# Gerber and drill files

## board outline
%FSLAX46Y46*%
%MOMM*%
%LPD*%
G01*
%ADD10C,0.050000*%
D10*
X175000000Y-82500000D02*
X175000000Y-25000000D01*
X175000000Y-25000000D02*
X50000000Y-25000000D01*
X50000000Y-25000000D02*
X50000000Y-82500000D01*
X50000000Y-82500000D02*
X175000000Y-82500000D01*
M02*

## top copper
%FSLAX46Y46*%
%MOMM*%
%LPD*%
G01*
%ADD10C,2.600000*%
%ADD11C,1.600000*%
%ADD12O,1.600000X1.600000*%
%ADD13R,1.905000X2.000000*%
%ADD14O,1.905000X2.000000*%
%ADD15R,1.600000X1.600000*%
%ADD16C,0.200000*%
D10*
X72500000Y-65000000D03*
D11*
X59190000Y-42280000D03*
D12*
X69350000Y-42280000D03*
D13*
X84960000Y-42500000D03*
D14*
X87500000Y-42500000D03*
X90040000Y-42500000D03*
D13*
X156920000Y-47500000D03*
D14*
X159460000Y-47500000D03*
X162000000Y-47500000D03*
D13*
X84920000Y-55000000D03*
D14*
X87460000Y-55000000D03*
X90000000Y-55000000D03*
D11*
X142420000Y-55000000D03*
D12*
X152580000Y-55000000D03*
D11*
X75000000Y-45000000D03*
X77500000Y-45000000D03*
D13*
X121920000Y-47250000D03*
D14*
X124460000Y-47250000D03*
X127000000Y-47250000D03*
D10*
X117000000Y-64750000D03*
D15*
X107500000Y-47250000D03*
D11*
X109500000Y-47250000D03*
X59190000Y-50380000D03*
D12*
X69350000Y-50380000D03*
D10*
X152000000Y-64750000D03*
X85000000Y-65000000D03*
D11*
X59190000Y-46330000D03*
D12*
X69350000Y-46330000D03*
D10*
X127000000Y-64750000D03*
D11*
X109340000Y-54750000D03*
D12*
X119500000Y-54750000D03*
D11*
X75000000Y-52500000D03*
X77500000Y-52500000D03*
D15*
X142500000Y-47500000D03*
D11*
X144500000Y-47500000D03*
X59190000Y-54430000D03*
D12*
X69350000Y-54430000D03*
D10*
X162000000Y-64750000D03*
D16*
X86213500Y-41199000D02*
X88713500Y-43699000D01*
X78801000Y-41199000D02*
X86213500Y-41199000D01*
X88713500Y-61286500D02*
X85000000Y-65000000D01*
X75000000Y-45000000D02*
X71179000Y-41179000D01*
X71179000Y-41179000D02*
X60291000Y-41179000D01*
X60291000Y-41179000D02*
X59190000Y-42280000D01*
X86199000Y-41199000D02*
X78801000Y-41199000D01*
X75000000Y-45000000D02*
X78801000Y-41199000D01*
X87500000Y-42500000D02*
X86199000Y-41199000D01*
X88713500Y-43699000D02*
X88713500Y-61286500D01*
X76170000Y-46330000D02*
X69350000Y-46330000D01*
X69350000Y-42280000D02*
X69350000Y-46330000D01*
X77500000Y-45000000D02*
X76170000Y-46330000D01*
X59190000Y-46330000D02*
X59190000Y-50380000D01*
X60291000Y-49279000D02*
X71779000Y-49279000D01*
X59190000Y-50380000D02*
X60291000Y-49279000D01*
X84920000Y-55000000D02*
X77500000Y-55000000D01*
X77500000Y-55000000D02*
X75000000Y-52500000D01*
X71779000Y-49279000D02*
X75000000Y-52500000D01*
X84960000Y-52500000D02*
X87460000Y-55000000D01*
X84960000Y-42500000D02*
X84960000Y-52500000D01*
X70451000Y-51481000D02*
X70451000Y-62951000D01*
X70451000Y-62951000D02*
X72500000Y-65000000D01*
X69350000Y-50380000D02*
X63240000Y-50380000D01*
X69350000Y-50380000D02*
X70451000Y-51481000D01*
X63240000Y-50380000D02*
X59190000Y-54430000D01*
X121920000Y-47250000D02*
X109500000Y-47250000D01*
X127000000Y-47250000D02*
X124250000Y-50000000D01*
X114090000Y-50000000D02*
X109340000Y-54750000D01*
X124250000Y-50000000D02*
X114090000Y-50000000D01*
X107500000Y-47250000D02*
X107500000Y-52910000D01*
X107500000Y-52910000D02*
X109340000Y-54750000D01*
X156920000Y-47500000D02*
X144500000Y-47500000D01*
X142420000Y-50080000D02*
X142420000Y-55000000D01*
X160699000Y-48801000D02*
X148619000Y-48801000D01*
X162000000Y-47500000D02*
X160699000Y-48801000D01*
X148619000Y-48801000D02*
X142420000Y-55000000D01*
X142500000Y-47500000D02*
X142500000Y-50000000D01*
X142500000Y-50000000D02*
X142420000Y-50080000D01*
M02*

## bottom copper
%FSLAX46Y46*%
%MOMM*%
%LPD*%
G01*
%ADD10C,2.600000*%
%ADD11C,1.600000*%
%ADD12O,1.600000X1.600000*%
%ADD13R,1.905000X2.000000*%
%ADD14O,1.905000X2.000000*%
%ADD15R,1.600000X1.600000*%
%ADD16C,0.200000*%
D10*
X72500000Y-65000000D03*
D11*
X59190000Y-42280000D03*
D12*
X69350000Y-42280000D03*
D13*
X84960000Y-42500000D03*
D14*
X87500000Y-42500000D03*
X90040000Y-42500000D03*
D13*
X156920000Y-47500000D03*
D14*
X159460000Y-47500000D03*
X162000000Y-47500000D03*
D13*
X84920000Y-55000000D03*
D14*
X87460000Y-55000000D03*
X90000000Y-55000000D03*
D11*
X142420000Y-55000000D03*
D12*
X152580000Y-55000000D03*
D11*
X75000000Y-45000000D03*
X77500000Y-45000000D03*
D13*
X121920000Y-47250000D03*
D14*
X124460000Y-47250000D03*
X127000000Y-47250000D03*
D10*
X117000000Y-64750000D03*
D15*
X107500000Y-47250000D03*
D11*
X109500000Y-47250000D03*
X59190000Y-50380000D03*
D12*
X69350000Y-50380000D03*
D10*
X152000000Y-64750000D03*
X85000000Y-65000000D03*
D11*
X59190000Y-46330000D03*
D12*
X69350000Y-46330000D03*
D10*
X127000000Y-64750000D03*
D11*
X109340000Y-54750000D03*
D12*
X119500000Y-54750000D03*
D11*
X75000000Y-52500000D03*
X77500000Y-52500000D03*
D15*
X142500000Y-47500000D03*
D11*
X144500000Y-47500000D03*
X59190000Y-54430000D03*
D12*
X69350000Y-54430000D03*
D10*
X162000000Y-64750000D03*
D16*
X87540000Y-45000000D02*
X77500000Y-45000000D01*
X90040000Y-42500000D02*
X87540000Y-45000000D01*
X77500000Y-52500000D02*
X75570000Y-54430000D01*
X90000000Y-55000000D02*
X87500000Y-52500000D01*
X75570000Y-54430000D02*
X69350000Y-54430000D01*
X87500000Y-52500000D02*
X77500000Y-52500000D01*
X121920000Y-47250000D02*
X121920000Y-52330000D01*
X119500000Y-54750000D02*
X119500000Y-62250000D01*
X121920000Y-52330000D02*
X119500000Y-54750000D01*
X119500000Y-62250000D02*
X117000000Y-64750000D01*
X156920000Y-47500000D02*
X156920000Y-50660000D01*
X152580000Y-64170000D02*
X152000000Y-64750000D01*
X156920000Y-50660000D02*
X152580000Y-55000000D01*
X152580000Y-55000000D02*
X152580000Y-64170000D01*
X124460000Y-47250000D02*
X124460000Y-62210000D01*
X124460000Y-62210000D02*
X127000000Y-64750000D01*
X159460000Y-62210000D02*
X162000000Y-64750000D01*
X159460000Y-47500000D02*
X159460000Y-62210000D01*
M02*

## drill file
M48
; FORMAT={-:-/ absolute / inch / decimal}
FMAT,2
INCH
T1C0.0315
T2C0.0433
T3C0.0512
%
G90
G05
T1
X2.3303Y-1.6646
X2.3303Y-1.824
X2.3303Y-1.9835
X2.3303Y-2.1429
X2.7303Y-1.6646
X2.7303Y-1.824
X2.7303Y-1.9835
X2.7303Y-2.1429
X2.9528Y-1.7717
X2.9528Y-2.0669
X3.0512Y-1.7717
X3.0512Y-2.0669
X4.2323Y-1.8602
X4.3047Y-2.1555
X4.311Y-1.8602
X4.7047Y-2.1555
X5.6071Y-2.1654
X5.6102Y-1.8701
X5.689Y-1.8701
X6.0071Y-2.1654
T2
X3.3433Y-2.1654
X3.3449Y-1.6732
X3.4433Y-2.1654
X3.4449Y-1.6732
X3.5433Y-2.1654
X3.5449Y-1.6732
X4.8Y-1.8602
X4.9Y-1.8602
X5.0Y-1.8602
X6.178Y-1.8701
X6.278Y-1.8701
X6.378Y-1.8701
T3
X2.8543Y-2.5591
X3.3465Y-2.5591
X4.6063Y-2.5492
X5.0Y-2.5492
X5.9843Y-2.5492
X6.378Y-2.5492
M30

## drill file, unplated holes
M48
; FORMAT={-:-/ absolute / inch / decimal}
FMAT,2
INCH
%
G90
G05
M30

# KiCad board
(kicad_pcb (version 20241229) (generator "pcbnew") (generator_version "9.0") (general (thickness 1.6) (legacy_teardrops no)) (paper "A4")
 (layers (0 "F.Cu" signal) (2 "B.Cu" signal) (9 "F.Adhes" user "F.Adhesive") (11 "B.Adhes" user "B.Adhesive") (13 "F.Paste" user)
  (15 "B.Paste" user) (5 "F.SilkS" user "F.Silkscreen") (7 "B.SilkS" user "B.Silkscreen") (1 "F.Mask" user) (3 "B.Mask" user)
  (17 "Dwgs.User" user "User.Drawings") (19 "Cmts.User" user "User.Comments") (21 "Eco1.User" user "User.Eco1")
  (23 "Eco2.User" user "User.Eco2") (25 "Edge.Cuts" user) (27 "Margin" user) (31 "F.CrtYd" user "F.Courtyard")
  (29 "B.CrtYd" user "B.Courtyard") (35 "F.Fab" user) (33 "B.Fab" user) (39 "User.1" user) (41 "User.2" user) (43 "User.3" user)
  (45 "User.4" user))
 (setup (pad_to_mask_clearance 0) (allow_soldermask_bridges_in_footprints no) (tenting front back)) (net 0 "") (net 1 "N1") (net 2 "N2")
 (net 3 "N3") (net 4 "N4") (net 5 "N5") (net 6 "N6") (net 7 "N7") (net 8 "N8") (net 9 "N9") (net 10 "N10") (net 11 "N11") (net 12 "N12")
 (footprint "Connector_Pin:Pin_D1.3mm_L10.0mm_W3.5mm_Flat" (layer "F.Cu") (at 72.5 65)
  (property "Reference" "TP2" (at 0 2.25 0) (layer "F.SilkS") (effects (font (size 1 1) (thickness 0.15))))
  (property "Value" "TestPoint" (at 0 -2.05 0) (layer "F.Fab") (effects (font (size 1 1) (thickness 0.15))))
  (pad "1" thru_hole circle (at 0 0) (size 2.6 2.6) (drill 1.3) (layers "*.Cu" "*.Mask") (remove_unused_layers no) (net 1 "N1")))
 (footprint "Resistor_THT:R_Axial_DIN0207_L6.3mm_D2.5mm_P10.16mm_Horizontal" (layer "F.Cu") (at 59.19 42.28)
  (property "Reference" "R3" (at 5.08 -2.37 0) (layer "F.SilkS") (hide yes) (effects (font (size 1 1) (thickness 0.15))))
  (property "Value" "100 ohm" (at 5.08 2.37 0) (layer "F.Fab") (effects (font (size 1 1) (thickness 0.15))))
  (pad "1" thru_hole circle (at 0 0) (size 1.6 1.6) (drill 0.8) (layers "*.Cu" "*.Mask") (remove_unused_layers no) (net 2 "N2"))
  (pad "2" thru_hole oval (at 10.16 0) (size 1.6 1.6) (drill 0.8) (layers "*.Cu" "*.Mask") (remove_unused_layers no) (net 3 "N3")))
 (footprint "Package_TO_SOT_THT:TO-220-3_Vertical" (layer "F.Cu") (at 84.96 42.5)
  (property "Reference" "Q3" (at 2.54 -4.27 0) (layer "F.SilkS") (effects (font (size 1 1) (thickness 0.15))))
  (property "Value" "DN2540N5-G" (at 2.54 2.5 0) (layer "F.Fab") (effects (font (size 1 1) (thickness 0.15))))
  (pad "1" thru_hole rect (at 0 0) (size 1.905 2) (drill 1.1) (layers "*.Cu" "*.Mask") (remove_unused_layers no) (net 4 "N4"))
  (pad "2" thru_hole oval (at 2.54 0) (size 1.905 2) (drill 1.1) (layers "*.Cu" "*.Mask") (remove_unused_layers no) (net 2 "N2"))
  (pad "3" thru_hole oval (at 5.08 0) (size 1.905 2) (drill 1.1) (layers "*.Cu" "*.Mask") (remove_unused_layers no) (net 3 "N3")))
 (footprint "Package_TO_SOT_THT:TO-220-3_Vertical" (layer "F.Cu") (at 156.92 47.5)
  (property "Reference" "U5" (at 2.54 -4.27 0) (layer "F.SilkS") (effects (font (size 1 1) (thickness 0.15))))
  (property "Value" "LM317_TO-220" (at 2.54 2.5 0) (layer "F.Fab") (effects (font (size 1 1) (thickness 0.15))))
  (pad "1" thru_hole rect (at 0 0) (size 1.905 2) (drill 1.1) (layers "*.Cu" "*.Mask") (remove_unused_layers no) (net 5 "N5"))
  (pad "2" thru_hole oval (at 2.54 0) (size 1.905 2) (drill 1.1) (layers "*.Cu" "*.Mask") (remove_unused_layers no) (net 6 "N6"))
  (pad "3" thru_hole oval (at 5.08 0) (size 1.905 2) (drill 1.1) (layers "*.Cu" "*.Mask") (remove_unused_layers no) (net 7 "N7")))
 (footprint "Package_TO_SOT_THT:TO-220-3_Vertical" (layer "F.Cu") (at 84.92 55)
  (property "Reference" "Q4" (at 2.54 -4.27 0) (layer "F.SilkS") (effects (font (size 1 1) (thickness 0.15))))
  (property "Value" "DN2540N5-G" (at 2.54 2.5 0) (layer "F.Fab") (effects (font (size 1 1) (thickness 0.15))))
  (pad "1" thru_hole rect (at 0 0) (size 1.905 2) (drill 1.1) (layers "*.Cu" "*.Mask") (remove_unused_layers no) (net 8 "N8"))
  (pad "2" thru_hole oval (at 2.54 0) (size 1.905 2) (drill 1.1) (layers "*.Cu" "*.Mask") (remove_unused_layers no) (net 4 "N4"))
  (pad "3" thru_hole oval (at 5.08 0) (size 1.905 2) (drill 1.1) (layers "*.Cu" "*.Mask") (remove_unused_layers no) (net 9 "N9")))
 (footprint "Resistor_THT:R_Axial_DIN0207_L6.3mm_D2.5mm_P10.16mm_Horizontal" (layer "F.Cu") (at 142.42 55)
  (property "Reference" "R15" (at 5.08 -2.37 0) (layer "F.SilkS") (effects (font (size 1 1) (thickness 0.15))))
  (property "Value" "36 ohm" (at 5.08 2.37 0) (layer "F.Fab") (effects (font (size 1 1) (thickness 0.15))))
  (pad "1" thru_hole circle (at 0 0) (size 1.6 1.6) (drill 0.8) (layers "*.Cu" "*.Mask") (remove_unused_layers no) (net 7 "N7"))
  (pad "2" thru_hole oval (at 10.16 0) (size 1.6 1.6) (drill 0.8) (layers "*.Cu" "*.Mask") (remove_unused_layers no) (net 5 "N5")))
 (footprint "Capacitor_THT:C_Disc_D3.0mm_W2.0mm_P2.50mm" (layer "F.Cu") (at 75 45)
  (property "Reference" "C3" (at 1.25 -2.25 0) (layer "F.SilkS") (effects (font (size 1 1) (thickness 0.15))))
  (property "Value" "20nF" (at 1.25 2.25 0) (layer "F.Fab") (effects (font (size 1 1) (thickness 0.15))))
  (pad "1" thru_hole circle (at 0 0) (size 1.6 1.6) (drill 0.8) (layers "*.Cu" "*.Mask") (remove_unused_layers no) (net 2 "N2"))
  (pad "2" thru_hole circle (at 2.5 0) (size 1.6 1.6) (drill 0.8) (layers "*.Cu" "*.Mask") (remove_unused_layers no) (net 3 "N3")))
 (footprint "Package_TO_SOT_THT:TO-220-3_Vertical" (layer "F.Cu") (at 121.92 47.25)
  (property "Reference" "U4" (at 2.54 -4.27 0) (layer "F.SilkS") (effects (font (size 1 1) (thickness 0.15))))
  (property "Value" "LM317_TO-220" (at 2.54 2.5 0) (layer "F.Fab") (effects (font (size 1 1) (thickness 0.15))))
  (pad "1" thru_hole rect (at 0 0) (size 1.905 2) (drill 1.1) (layers "*.Cu" "*.Mask") (remove_unused_layers no) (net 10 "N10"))
  (pad "2" thru_hole oval (at 2.54 0) (size 1.905 2) (drill 1.1) (layers "*.Cu" "*.Mask") (remove_unused_layers no) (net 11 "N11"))
  (pad "3" thru_hole oval (at 5.08 0) (size 1.905 2) (drill 1.1) (layers "*.Cu" "*.Mask") (remove_unused_layers no) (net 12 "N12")))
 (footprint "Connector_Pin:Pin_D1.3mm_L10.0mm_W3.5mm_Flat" (layer "F.Cu") (at 117 64.75)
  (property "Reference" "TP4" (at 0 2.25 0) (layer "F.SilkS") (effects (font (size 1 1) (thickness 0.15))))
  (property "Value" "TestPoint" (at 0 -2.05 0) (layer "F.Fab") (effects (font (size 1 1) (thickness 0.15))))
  (pad "1" thru_hole circle (at 0 0) (size 2.6 2.6) (drill 1.3) (layers "*.Cu" "*.Mask") (remove_unused_layers no) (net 10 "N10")))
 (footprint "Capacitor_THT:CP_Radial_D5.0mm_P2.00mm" (layer "F.Cu") (at 107.5 47.25)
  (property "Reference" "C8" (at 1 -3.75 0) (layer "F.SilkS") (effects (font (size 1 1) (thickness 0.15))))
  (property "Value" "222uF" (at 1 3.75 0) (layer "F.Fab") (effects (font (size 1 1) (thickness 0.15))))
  (pad "1" thru_hole rect (at 0 0) (size 1.6 1.6) (drill 0.8) (layers "*.Cu" "*.Mask") (remove_unused_layers no) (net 12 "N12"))
  (pad "2" thru_hole circle (at 2 0) (size 1.6 1.6) (drill 0.8) (layers "*.Cu" "*.Mask") (remove_unused_layers no) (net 10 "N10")))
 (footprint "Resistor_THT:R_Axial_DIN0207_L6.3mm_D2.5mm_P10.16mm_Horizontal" (layer "F.Cu") (at 59.19 50.38)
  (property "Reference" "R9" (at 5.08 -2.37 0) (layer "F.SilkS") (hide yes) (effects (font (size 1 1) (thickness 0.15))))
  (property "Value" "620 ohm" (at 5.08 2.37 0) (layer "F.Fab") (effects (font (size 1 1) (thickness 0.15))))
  (pad "1" thru_hole circle (at 0 0) (size 1.6 1.6) (drill 0.8) (layers "*.Cu" "*.Mask") (remove_unused_layers no) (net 8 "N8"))
  (pad "2" thru_hole oval (at 10.16 0) (size 1.6 1.6) (drill 0.8) (layers "*.Cu" "*.Mask") (remove_unused_layers no) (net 1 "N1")))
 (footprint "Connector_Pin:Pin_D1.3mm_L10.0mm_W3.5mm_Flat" (layer "F.Cu") (at 152 64.75)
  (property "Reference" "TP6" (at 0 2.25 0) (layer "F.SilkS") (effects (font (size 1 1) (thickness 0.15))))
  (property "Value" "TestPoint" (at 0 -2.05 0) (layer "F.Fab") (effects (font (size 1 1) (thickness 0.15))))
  (pad "1" thru_hole circle (at 0 0) (size 2.6 2.6) (drill 1.3) (layers "*.Cu" "*.Mask") (remove_unused_layers no) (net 5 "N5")))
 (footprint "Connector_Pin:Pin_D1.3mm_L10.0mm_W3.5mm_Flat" (layer "F.Cu") (at 85 65)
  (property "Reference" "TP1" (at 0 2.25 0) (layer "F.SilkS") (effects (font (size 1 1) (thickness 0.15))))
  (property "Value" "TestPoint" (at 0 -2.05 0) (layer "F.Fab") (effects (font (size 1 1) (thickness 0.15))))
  (pad "1" thru_hole circle (at 0 0) (size 2.6 2.6) (drill 1.3) (layers "*.Cu" "*.Mask") (remove_unused_layers no) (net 2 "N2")))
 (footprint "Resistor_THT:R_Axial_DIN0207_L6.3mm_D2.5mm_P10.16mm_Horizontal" (layer "F.Cu") (at 59.19 46.33)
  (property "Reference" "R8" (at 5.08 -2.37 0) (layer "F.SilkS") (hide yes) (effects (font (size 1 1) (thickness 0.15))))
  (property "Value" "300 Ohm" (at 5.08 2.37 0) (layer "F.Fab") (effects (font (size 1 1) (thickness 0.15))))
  (pad "1" thru_hole circle (at 0 0) (size 1.6 1.6) (drill 0.8) (layers "*.Cu" "*.Mask") (remove_unused_layers no) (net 8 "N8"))
  (pad "2" thru_hole oval (at 10.16 0) (size 1.6 1.6) (drill 0.8) (layers "*.Cu" "*.Mask") (remove_unused_layers no) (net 3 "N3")))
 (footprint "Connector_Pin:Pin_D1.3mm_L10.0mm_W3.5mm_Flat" (layer "F.Cu") (at 127 64.75)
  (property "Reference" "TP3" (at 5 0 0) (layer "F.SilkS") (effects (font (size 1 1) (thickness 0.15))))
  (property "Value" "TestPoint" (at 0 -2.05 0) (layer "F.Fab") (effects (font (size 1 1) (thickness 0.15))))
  (pad "1" thru_hole circle (at 0 0) (size 2.6 2.6) (drill 1.3) (layers "*.Cu" "*.Mask") (remove_unused_layers no) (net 11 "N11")))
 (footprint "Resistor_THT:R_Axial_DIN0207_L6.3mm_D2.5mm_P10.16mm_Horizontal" (layer "F.Cu") (at 109.34 54.75)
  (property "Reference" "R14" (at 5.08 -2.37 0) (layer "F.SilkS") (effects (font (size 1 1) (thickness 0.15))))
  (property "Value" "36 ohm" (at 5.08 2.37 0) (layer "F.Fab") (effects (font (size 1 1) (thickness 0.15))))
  (pad "1" thru_hole circle (at 0 0) (size 1.6 1.6) (drill 0.8) (layers "*.Cu" "*.Mask") (remove_unused_layers no) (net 12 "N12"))
  (pad "2" thru_hole oval (at 10.16 0) (size 1.6 1.6) (drill 0.8) (layers "*.Cu" "*.Mask") (remove_unused_layers no) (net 10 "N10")))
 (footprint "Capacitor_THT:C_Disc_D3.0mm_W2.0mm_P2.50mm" (layer "F.Cu") (at 75 52.5)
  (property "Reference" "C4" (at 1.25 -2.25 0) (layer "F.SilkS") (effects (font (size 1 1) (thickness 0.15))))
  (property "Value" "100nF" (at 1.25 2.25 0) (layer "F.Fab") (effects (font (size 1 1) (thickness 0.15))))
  (pad "1" thru_hole circle (at 0 0) (size 1.6 1.6) (drill 0.8) (layers "*.Cu" "*.Mask") (remove_unused_layers no) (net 8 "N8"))
  (pad "2" thru_hole circle (at 2.5 0) (size 1.6 1.6) (drill 0.8) (layers "*.Cu" "*.Mask") (remove_unused_layers no) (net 9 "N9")))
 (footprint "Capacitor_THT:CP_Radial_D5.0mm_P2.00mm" (layer "F.Cu") (at 142.5 47.5)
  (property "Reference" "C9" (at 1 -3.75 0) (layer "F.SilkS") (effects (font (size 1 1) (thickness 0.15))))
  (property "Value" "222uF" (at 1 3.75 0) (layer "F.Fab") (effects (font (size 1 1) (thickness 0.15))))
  (pad "1" thru_hole rect (at 0 0) (size 1.6 1.6) (drill 0.8) (layers "*.Cu" "*.Mask") (remove_unused_layers no) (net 7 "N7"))
  (pad "2" thru_hole circle (at 2 0) (size 1.6 1.6) (drill 0.8) (layers "*.Cu" "*.Mask") (remove_unused_layers no) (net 5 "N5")))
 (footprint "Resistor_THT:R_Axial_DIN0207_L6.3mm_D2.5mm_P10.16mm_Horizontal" (layer "F.Cu") (at 59.19 54.43)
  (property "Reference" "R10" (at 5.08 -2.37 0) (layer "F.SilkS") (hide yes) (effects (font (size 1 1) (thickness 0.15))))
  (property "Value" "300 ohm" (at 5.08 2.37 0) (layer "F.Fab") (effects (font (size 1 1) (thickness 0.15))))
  (pad "1" thru_hole circle (at 0 0) (size 1.6 1.6) (drill 0.8) (layers "*.Cu" "*.Mask") (remove_unused_layers no) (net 1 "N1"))
  (pad "2" thru_hole oval (at 10.16 0) (size 1.6 1.6) (drill 0.8) (layers "*.Cu" "*.Mask") (remove_unused_layers no) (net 9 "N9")))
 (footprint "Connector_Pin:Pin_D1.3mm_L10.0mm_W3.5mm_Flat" (layer "F.Cu") (at 162 64.75)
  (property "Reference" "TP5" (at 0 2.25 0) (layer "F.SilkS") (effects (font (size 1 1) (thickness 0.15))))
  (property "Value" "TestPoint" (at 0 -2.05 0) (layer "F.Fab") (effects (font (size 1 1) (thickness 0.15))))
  (pad "1" thru_hole circle (at 0 0) (size 2.6 2.6) (drill 1.3) (layers "*.Cu" "*.Mask") (remove_unused_layers no) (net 6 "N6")))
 (gr_line (start 175 82.5) (end 175 25) (stroke (width 0.05) (type default)) (layer "Edge.Cuts"))
 (gr_line (start 175 25) (end 50 25) (stroke (width 0.05) (type default)) (layer "Edge.Cuts"))
 (gr_line (start 50 25) (end 50 82.5) (stroke (width 0.05) (type default)) (layer "Edge.Cuts"))
 (gr_line (start 50 82.5) (end 175 82.5) (stroke (width 0.05) (type default)) (layer "Edge.Cuts"))
 (segment (start 86.2135 41.199) (end 88.7135 43.699) (width 0.2) (layer "F.Cu") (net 2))
 (segment (start 78.801 41.199) (end 86.2135 41.199) (width 0.2) (layer "F.Cu") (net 2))
 (segment (start 88.7135 61.2865) (end 85 65) (width 0.2) (layer "F.Cu") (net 2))
 (segment (start 75 45) (end 71.179 41.179) (width 0.2) (layer "F.Cu") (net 2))
 (segment (start 71.179 41.179) (end 60.291 41.179) (width 0.2) (layer "F.Cu") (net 2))
 (segment (start 60.291 41.179) (end 59.19 42.28) (width 0.2) (layer "F.Cu") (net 2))
 (segment (start 86.199 41.199) (end 78.801 41.199) (width 0.2) (layer "F.Cu") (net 2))
 (segment (start 75 45) (end 78.801 41.199) (width 0.2) (layer "F.Cu") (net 2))
 (segment (start 87.5 42.5) (end 86.199 41.199) (width 0.2) (layer "F.Cu") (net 2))
 (segment (start 88.7135 43.699) (end 88.7135 61.2865) (width 0.2) (layer "F.Cu") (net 2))
 (segment (start 76.17 46.33) (end 69.35 46.33) (width 0.2) (layer "F.Cu") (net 3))
 (segment (start 69.35 42.28) (end 69.35 46.33) (width 0.2) (layer "F.Cu") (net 3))
 (segment (start 77.5 45) (end 76.17 46.33) (width 0.2) (layer "F.Cu") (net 3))
 (segment (start 87.54 45) (end 77.5 45) (width 0.2) (layer "B.Cu") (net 3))
 (segment (start 90.04 42.5) (end 87.54 45) (width 0.2) (layer "B.Cu") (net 3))
 (segment (start 59.19 46.33) (end 59.19 50.38) (width 0.2) (layer "F.Cu") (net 8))
 (segment (start 60.291 49.279) (end 71.779 49.279) (width 0.2) (layer "F.Cu") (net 8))
 (segment (start 59.19 50.38) (end 60.291 49.279) (width 0.2) (layer "F.Cu") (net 8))
 (segment (start 84.92 55) (end 77.5 55) (width 0.2) (layer "F.Cu") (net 8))
 (segment (start 77.5 55) (end 75 52.5) (width 0.2) (layer "F.Cu") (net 8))
 (segment (start 71.779 49.279) (end 75 52.5) (width 0.2) (layer "F.Cu") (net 8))
 (segment (start 77.5 52.5) (end 75.57 54.43) (width 0.2) (layer "B.Cu") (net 9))
 (segment (start 90 55) (end 87.5 52.5) (width 0.2) (layer "B.Cu") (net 9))
 (segment (start 75.57 54.43) (end 69.35 54.43) (width 0.2) (layer "B.Cu") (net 9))
 (segment (start 87.5 52.5) (end 77.5 52.5) (width 0.2) (layer "B.Cu") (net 9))
 (segment (start 84.96 52.5) (end 87.46 55) (width 0.2) (layer "F.Cu") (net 4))
 (segment (start 84.96 42.5) (end 84.96 52.5) (width 0.2) (layer "F.Cu") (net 4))
 (segment (start 70.451 51.481) (end 70.451 62.951) (width 0.2) (layer "F.Cu") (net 1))
 (segment (start 70.451 62.951) (end 72.5 65) (width 0.2) (layer "F.Cu") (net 1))
 (segment (start 69.35 50.38) (end 63.24 50.38) (width 0.2) (layer "F.Cu") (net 1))
 (segment (start 69.35 50.38) (end 70.451 51.481) (width 0.2) (layer "F.Cu") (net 1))
 (segment (start 63.24 50.38) (end 59.19 54.43) (width 0.2) (layer "F.Cu") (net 1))
 (segment (start 121.92 47.25) (end 109.5 47.25) (width 0.2) (layer "F.Cu") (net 10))
 (segment (start 121.92 47.25) (end 121.92 52.33) (width 0.2) (layer "B.Cu") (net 10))
 (segment (start 119.5 54.75) (end 119.5 62.25) (width 0.2) (layer "B.Cu") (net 10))
 (segment (start 121.92 52.33) (end 119.5 54.75) (width 0.2) (layer "B.Cu") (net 10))
 (segment (start 119.5 62.25) (end 117 64.75) (width 0.2) (layer "B.Cu") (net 10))
 (segment (start 127 47.25) (end 124.25 50) (width 0.2) (layer "F.Cu") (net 12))
 (segment (start 114.09 50) (end 109.34 54.75) (width 0.2) (layer "F.Cu") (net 12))
 (segment (start 124.25 50) (end 114.09 50) (width 0.2) (layer "F.Cu") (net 12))
 (segment (start 107.5 47.25) (end 107.5 52.91) (width 0.2) (layer "F.Cu") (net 12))
 (segment (start 107.5 52.91) (end 109.34 54.75) (width 0.2) (layer "F.Cu") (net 12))
 (segment (start 156.92 47.5) (end 144.5 47.5) (width 0.2) (layer "F.Cu") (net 5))
 (segment (start 156.92 47.5) (end 156.92 50.66) (width 0.2) (layer "B.Cu") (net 5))
 (segment (start 152.58 64.17) (end 152 64.75) (width 0.2) (layer "B.Cu") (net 5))
 (segment (start 156.92 50.66) (end 152.58 55) (width 0.2) (layer "B.Cu") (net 5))
 (segment (start 152.58 55) (end 152.58 64.17) (width 0.2) (layer "B.Cu") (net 5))
 (segment (start 142.42 50.08) (end 142.42 55) (width 0.2) (layer "F.Cu") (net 7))
 (segment (start 160.699 48.801) (end 148.619 48.801) (width 0.2) (layer "F.Cu") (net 7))
 (segment (start 162 47.5) (end 160.699 48.801) (width 0.2) (layer "F.Cu") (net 7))
 (segment (start 148.619 48.801) (end 142.42 55) (width 0.2) (layer "F.Cu") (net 7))
 (segment (start 142.5 47.5) (end 142.5 50) (width 0.2) (layer "F.Cu") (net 7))
 (segment (start 142.5 50) (end 142.42 50.08) (width 0.2) (layer "F.Cu") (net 7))
 (segment (start 124.46 47.25) (end 124.46 62.21) (width 0.2) (layer "B.Cu") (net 11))
 (segment (start 124.46 62.21) (end 127 64.75) (width 0.2) (layer "B.Cu") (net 11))
 (segment (start 159.46 62.21) (end 162 64.75) (width 0.2) (layer "B.Cu") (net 6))
 (segment (start 159.46 47.5) (end 159.46 62.21) (width 0.2) (layer "B.Cu") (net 6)))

